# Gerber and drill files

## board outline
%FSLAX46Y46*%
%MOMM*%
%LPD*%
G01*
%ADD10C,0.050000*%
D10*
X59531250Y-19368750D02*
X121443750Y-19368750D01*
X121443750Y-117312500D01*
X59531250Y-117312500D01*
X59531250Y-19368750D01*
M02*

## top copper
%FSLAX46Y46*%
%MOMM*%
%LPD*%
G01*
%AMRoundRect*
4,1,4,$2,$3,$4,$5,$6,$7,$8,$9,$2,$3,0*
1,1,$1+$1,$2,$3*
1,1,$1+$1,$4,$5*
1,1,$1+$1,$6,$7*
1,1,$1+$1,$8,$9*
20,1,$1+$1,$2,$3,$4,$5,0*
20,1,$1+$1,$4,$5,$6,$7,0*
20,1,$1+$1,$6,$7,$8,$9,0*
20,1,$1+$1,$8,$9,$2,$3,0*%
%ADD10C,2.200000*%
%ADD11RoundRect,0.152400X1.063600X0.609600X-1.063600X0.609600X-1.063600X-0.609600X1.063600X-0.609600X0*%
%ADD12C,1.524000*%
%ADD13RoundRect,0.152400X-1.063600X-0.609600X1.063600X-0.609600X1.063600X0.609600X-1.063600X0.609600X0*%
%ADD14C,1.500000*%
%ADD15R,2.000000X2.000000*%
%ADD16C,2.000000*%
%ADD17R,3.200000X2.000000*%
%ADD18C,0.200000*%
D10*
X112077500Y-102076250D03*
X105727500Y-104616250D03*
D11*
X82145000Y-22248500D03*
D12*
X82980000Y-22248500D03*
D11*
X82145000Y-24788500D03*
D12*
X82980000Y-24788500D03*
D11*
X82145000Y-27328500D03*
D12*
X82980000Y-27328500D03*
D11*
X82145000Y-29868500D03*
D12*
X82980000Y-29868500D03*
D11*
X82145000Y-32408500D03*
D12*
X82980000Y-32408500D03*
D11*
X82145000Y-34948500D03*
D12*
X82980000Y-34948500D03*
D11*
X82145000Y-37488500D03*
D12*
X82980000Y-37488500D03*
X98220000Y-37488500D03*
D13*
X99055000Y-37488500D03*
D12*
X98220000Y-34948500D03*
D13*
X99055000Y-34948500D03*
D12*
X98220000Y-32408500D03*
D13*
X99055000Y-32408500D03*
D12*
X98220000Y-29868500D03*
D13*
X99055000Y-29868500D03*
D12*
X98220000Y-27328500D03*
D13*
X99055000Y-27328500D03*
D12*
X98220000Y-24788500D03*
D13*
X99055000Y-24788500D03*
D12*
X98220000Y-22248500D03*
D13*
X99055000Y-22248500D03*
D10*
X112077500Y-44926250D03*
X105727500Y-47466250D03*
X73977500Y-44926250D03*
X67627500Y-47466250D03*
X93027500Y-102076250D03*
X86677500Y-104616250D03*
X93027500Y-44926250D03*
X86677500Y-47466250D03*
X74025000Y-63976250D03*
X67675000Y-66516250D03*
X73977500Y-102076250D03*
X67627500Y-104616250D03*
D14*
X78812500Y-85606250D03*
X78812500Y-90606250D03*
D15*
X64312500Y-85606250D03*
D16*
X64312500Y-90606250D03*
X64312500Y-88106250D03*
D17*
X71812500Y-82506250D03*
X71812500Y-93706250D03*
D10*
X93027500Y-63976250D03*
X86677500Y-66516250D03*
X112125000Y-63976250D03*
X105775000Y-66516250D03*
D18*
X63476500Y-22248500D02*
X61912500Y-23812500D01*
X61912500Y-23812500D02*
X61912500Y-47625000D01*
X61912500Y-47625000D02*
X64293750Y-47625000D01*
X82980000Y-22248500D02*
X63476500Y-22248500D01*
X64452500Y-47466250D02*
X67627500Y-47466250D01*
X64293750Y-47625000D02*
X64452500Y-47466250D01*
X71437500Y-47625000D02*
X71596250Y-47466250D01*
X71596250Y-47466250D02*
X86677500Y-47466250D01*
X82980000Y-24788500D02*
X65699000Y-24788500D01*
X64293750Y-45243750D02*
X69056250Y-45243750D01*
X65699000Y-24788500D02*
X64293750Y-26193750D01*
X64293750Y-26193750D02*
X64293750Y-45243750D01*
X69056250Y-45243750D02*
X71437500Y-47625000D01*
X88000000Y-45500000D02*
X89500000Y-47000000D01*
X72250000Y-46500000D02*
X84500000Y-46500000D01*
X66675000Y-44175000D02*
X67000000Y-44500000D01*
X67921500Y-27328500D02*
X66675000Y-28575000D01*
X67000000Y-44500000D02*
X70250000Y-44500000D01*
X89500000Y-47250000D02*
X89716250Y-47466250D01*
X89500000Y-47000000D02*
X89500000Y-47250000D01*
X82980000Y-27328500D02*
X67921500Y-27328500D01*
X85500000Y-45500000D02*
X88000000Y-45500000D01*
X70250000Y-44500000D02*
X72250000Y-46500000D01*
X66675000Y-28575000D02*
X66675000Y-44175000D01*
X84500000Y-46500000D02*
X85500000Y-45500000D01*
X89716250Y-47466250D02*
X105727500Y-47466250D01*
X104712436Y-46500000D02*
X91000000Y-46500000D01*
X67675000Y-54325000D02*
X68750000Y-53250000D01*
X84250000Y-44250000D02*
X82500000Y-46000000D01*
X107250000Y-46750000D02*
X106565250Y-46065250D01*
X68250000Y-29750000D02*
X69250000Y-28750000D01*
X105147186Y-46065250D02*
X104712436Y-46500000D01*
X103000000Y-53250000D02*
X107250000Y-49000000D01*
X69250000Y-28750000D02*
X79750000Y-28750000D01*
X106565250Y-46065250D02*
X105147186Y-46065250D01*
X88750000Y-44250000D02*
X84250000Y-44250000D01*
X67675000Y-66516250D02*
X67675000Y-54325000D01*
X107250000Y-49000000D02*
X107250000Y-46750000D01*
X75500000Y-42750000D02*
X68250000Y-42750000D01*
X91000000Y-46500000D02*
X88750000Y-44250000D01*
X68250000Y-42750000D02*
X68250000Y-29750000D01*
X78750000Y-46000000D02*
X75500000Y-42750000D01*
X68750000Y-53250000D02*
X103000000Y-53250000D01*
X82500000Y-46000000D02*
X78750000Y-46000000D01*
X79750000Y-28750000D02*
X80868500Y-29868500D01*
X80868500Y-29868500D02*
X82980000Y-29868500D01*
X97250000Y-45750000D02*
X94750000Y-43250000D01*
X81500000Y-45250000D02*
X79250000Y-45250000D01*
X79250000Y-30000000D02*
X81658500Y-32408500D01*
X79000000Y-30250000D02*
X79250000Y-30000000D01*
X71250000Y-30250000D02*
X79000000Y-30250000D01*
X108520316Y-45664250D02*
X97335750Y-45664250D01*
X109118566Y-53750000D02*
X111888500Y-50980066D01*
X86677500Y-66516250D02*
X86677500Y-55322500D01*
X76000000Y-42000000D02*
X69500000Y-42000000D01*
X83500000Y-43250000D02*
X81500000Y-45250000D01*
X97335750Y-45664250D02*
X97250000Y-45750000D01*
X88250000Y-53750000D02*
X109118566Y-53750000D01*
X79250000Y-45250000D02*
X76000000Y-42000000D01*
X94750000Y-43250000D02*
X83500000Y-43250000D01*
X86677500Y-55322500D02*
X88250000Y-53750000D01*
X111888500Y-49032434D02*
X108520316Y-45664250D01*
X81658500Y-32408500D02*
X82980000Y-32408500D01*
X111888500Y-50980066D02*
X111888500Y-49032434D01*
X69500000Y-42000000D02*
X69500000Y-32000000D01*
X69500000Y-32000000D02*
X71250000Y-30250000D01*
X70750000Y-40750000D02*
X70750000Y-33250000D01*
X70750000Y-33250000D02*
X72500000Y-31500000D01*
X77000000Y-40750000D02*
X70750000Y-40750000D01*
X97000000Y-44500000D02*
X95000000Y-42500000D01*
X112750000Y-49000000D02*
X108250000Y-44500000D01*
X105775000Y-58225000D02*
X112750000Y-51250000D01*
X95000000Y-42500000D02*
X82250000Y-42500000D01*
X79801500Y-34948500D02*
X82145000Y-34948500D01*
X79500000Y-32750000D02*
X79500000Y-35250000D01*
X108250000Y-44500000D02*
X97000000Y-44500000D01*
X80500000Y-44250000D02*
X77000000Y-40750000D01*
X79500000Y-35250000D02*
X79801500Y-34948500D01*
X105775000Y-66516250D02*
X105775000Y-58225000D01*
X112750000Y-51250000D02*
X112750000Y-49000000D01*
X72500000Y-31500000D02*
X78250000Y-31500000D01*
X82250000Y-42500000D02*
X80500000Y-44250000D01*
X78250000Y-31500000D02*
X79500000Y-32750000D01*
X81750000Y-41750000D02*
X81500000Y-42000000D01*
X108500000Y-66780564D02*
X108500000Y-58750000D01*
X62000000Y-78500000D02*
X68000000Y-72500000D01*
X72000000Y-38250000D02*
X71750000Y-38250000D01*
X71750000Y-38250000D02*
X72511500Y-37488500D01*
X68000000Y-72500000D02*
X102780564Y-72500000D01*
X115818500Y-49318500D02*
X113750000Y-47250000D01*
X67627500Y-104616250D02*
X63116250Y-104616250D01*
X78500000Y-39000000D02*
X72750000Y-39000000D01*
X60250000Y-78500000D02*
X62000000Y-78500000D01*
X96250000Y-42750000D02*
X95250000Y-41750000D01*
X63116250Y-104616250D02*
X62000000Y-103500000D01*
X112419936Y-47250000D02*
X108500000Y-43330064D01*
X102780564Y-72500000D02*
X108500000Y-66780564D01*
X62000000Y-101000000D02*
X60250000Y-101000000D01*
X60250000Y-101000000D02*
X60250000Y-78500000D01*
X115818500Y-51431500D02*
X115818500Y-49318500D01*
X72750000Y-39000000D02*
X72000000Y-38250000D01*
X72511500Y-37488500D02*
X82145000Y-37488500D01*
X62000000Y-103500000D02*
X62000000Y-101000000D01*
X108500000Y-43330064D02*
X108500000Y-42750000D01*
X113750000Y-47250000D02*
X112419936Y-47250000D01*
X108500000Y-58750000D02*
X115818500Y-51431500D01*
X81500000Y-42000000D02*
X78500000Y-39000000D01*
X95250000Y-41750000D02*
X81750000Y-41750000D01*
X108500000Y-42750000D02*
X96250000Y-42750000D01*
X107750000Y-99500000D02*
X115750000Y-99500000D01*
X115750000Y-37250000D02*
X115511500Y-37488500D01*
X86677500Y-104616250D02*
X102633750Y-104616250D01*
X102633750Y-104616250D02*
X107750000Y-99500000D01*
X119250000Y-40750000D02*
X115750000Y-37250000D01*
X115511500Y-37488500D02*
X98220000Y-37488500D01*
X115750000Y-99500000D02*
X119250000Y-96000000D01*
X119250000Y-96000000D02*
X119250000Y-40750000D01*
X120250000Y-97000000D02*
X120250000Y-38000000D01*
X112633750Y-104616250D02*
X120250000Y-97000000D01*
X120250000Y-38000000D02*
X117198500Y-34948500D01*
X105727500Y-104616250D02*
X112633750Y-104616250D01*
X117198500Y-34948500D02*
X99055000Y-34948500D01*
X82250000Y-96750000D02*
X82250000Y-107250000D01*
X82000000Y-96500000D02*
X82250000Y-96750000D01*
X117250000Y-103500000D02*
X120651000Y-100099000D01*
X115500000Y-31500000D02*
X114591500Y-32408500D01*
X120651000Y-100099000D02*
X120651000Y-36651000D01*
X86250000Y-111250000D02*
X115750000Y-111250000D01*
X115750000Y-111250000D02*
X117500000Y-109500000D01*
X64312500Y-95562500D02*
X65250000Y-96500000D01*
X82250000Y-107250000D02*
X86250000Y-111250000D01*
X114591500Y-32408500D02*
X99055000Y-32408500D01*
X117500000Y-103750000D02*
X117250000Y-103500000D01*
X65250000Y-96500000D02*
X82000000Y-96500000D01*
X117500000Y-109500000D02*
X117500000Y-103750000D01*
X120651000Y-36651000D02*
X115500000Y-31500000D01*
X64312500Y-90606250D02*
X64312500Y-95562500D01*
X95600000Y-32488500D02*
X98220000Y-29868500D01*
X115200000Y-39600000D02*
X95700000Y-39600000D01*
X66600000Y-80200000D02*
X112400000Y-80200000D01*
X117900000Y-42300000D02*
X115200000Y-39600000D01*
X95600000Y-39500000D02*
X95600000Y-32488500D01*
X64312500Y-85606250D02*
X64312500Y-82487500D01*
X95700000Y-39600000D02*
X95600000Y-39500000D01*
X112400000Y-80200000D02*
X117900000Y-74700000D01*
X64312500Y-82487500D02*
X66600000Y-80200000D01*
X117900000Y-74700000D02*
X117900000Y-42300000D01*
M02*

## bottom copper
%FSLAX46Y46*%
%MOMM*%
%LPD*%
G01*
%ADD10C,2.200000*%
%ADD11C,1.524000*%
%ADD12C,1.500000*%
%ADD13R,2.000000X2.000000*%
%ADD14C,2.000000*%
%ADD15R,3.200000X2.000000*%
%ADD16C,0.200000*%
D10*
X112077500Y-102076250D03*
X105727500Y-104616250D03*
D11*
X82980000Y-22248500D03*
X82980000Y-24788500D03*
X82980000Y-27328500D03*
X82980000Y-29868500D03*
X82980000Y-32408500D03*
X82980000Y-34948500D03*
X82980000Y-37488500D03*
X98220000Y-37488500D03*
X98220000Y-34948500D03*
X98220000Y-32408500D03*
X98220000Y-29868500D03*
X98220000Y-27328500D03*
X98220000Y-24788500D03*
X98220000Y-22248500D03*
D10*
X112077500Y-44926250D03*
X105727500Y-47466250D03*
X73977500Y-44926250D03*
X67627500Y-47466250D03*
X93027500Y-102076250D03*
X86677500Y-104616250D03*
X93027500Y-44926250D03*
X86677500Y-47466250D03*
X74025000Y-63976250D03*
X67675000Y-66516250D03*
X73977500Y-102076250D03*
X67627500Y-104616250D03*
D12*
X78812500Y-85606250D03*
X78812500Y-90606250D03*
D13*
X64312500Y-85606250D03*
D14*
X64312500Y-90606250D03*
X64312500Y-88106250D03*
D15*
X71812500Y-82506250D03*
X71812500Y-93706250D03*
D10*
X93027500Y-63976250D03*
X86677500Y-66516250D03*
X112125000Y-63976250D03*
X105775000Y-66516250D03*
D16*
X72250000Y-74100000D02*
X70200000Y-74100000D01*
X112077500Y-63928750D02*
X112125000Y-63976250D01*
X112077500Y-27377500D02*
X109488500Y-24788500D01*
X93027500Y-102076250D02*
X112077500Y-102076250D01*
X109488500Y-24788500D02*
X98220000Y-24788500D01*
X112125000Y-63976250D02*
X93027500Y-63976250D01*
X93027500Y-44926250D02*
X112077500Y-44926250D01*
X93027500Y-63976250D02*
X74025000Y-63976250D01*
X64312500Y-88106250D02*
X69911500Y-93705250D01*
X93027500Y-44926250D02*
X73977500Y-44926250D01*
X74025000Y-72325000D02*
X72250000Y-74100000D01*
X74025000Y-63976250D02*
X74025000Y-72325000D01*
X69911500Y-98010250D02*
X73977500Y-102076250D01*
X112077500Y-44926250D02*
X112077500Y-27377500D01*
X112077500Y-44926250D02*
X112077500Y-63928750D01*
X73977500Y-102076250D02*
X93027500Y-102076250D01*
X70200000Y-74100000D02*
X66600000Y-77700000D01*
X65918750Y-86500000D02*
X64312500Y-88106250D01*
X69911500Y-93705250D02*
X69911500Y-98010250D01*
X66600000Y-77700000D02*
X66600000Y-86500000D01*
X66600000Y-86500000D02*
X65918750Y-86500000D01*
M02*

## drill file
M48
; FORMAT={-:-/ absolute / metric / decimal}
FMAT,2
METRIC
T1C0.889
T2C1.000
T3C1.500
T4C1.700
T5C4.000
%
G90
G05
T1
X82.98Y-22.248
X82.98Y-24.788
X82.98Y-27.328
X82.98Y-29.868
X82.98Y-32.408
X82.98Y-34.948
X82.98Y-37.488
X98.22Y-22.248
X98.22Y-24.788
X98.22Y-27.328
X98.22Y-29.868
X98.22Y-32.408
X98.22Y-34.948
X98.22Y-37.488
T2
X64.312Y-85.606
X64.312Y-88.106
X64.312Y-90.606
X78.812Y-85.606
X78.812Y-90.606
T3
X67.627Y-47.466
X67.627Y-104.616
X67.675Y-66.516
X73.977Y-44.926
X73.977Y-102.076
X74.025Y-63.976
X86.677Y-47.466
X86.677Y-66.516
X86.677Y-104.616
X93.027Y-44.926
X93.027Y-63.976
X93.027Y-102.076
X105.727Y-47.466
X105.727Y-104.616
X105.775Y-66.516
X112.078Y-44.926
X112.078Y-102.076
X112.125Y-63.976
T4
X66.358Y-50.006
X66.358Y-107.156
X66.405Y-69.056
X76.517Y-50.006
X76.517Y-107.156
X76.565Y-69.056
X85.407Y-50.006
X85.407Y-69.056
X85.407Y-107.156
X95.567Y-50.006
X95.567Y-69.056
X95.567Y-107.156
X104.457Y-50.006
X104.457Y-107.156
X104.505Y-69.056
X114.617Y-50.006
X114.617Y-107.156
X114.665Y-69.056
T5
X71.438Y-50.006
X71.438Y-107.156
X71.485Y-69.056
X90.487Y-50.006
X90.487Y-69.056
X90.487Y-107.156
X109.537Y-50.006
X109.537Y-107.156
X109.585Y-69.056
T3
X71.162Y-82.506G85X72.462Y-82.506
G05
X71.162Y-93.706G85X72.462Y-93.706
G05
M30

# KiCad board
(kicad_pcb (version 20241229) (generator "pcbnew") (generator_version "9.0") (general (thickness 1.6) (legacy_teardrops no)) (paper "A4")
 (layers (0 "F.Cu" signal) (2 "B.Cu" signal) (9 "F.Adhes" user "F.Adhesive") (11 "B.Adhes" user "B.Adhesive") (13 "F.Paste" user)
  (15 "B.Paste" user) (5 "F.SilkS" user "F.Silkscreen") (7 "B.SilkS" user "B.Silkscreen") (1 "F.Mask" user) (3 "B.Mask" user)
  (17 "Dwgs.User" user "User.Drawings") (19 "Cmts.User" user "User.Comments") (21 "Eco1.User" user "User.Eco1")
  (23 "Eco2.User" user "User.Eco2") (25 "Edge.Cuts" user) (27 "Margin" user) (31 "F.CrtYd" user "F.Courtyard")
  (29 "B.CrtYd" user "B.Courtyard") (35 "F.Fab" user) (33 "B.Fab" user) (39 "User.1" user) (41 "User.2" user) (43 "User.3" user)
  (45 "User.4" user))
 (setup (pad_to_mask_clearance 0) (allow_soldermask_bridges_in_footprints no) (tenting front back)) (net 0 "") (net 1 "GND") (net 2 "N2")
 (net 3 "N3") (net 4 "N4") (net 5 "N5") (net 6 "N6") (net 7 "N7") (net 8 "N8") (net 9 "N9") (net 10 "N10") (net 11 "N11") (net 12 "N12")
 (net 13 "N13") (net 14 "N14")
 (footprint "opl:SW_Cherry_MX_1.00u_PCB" (layer "F.Cu") (at 112.0775 102.07625)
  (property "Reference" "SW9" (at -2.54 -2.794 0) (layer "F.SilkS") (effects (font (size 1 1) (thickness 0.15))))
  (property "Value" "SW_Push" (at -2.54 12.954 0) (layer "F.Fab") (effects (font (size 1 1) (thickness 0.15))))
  (pad "" np_thru_hole circle (at -7.62 5.08) (size 1.7 1.7) (drill 1.7) (layers "*.Cu" "*.Mask"))
  (pad "" np_thru_hole circle (at -2.54 5.08) (size 4 4) (drill 4) (layers "*.Cu" "*.Mask"))
  (pad "" np_thru_hole circle (at 2.54 5.08) (size 1.7 1.7) (drill 1.7) (layers "*.Cu" "*.Mask"))
  (pad "1" thru_hole circle (at 0 0) (size 2.2 2.2) (drill 1.5) (layers "*.Cu" "*.Mask") (remove_unused_layers no) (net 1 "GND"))
  (pad "2" thru_hole circle (at -6.35 2.54) (size 2.2 2.2) (drill 1.5) (layers "*.Cu" "*.Mask") (remove_unused_layers no) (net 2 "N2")))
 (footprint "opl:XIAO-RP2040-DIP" (layer "F.Cu") (at 90.6 29.8685)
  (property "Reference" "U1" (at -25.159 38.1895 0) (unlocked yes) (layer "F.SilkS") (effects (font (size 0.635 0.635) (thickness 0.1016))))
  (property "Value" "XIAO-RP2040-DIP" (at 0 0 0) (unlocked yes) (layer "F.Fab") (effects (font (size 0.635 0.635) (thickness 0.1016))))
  (pad "1" smd roundrect (at -8.455 -7.62 180) (size 2.432 1.524) (layers "F.Cu" "F.Mask") (roundrect_rratio 0.1) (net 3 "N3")
   (thermal_bridge_angle 45))
  (pad "1" thru_hole circle (at -7.62 -7.62 180) (size 1.524 1.524) (drill 0.889) (layers "*.Cu" "*.Mask") (remove_unused_layers no)
   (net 3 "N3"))
  (pad "2" smd roundrect (at -8.455 -5.08 180) (size 2.432 1.524) (layers "F.Cu" "F.Mask") (roundrect_rratio 0.1) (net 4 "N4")
   (thermal_bridge_angle 45))
  (pad "2" thru_hole circle (at -7.62 -5.08 180) (size 1.524 1.524) (drill 0.889) (layers "*.Cu" "*.Mask") (remove_unused_layers no)
   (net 4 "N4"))
  (pad "3" smd roundrect (at -8.455 -2.54 180) (size 2.432 1.524) (layers "F.Cu" "F.Mask") (roundrect_rratio 0.1) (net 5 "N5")
   (thermal_bridge_angle 45))
  (pad "3" thru_hole circle (at -7.62 -2.54 180) (size 1.524 1.524) (drill 0.889) (layers "*.Cu" "*.Mask") (remove_unused_layers no)
   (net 5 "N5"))
  (pad "4" smd roundrect (at -8.455 0 180) (size 2.432 1.524) (layers "F.Cu" "F.Mask") (roundrect_rratio 0.1) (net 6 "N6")
   (thermal_bridge_angle 45))
  (pad "4" thru_hole circle (at -7.62 0 180) (size 1.524 1.524) (drill 0.889) (layers "*.Cu" "*.Mask") (remove_unused_layers no)
   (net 6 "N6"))
  (pad "5" smd roundrect (at -8.455 2.54 180) (size 2.432 1.524) (layers "F.Cu" "F.Mask") (roundrect_rratio 0.1) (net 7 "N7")
   (thermal_bridge_angle 45))
  (pad "5" thru_hole circle (at -7.62 2.54 180) (size 1.524 1.524) (drill 0.889) (layers "*.Cu" "*.Mask") (remove_unused_layers no)
   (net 7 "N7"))
  (pad "6" smd roundrect (at -8.455 5.08 180) (size 2.432 1.524) (layers "F.Cu" "F.Mask") (roundrect_rratio 0.1) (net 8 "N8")
   (thermal_bridge_angle 45))
  (pad "6" thru_hole circle (at -7.62 5.08 180) (size 1.524 1.524) (drill 0.889) (layers "*.Cu" "*.Mask") (remove_unused_layers no)
   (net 8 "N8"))
  (pad "7" smd roundrect (at -8.455 7.62 180) (size 2.432 1.524) (layers "F.Cu" "F.Mask") (roundrect_rratio 0.1) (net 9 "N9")
   (thermal_bridge_angle 45))
  (pad "7" thru_hole circle (at -7.62 7.62 180) (size 1.524 1.524) (drill 0.889) (layers "*.Cu" "*.Mask") (remove_unused_layers no)
   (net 9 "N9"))
  (pad "8" thru_hole circle (at 7.62 7.62) (size 1.524 1.524) (drill 0.889) (layers "*.Cu" "*.Mask") (remove_unused_layers no)
   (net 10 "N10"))
  (pad "8" smd roundrect (at 8.455 7.62) (size 2.432 1.524) (layers "F.Cu" "F.Mask") (roundrect_rratio 0.1) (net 10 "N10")
   (thermal_bridge_angle 45))
  (pad "9" thru_hole circle (at 7.62 5.08) (size 1.524 1.524) (drill 0.889) (layers "*.Cu" "*.Mask") (remove_unused_layers no) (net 2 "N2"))
  (pad "9" smd roundrect (at 8.455 5.08) (size 2.432 1.524) (layers "F.Cu" "F.Mask") (roundrect_rratio 0.1) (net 2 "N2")
   (thermal_bridge_angle 45))
  (pad "10" thru_hole circle (at 7.62 2.54) (size 1.524 1.524) (drill 0.889) (layers "*.Cu" "*.Mask") (remove_unused_layers no)
   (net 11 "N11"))
  (pad "10" smd roundrect (at 8.455 2.54) (size 2.432 1.524) (layers "F.Cu" "F.Mask") (roundrect_rratio 0.1) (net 11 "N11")
   (thermal_bridge_angle 45))
  (pad "11" thru_hole circle (at 7.62 0) (size 1.524 1.524) (drill 0.889) (layers "*.Cu" "*.Mask") (remove_unused_layers no) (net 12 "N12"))
  (pad "11" smd roundrect (at 8.455 0) (size 2.432 1.524) (layers "F.Cu" "F.Mask") (roundrect_rratio 0.1) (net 12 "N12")
   (thermal_bridge_angle 45))
  (pad "12" thru_hole circle (at 7.62 -2.54) (size 1.524 1.524) (drill 0.889) (layers "*.Cu" "*.Mask") (remove_unused_layers no)
   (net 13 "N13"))
  (pad "12" smd roundrect (at 8.455 -2.54) (size 2.432 1.524) (layers "F.Cu" "F.Mask") (roundrect_rratio 0.1) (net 13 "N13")
   (thermal_bridge_angle 45))
  (pad "13" thru_hole circle (at 7.62 -5.08) (size 1.524 1.524) (drill 0.889) (layers "*.Cu" "*.Mask") (remove_unused_layers no)
   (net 1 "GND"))
  (pad "13" smd roundrect (at 8.455 -5.08) (size 2.432 1.524) (layers "F.Cu" "F.Mask") (roundrect_rratio 0.1) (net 1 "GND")
   (thermal_bridge_angle 45))
  (pad "14" thru_hole circle (at 7.62 -7.62) (size 1.524 1.524) (drill 0.889) (layers "*.Cu" "*.Mask") (remove_unused_layers no)
   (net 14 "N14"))
  (pad "14" smd roundrect (at 8.455 -7.62) (size 2.432 1.524) (layers "F.Cu" "F.Mask") (roundrect_rratio 0.1) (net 14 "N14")
   (thermal_bridge_angle 45)))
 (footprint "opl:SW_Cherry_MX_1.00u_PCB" (layer "F.Cu") (at 112.0775 44.92625)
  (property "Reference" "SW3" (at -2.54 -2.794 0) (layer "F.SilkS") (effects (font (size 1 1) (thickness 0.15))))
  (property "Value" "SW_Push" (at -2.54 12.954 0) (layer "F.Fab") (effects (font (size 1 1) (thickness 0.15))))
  (pad "" np_thru_hole circle (at -7.62 5.08) (size 1.7 1.7) (drill 1.7) (layers "*.Cu" "*.Mask"))
  (pad "" np_thru_hole circle (at -2.54 5.08) (size 4 4) (drill 4) (layers "*.Cu" "*.Mask"))
  (pad "" np_thru_hole circle (at 2.54 5.08) (size 1.7 1.7) (drill 1.7) (layers "*.Cu" "*.Mask"))
  (pad "1" thru_hole circle (at 0 0) (size 2.2 2.2) (drill 1.5) (layers "*.Cu" "*.Mask") (remove_unused_layers no) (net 1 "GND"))
  (pad "2" thru_hole circle (at -6.35 2.54) (size 2.2 2.2) (drill 1.5) (layers "*.Cu" "*.Mask") (remove_unused_layers no) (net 5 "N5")))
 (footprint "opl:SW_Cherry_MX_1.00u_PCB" (layer "F.Cu") (at 73.9775 44.92625)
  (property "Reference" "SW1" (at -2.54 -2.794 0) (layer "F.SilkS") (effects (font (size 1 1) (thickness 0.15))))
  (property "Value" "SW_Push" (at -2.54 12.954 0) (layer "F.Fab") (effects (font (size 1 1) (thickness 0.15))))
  (pad "" np_thru_hole circle (at -7.62 5.08) (size 1.7 1.7) (drill 1.7) (layers "*.Cu" "*.Mask"))
  (pad "" np_thru_hole circle (at -2.54 5.08) (size 4 4) (drill 4) (layers "*.Cu" "*.Mask"))
  (pad "" np_thru_hole circle (at 2.54 5.08) (size 1.7 1.7) (drill 1.7) (layers "*.Cu" "*.Mask"))
  (pad "1" thru_hole circle (at 0 0) (size 2.2 2.2) (drill 1.5) (layers "*.Cu" "*.Mask") (remove_unused_layers no) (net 1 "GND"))
  (pad "2" thru_hole circle (at -6.35 2.54) (size 2.2 2.2) (drill 1.5) (layers "*.Cu" "*.Mask") (remove_unused_layers no) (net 3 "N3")))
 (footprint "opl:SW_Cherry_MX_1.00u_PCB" (layer "F.Cu") (at 93.0275 102.07625)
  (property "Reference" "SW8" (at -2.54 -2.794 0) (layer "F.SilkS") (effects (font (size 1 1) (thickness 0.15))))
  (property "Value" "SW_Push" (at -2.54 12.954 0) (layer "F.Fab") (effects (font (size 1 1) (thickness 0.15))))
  (pad "" np_thru_hole circle (at -7.62 5.08) (size 1.7 1.7) (drill 1.7) (layers "*.Cu" "*.Mask"))
  (pad "" np_thru_hole circle (at -2.54 5.08) (size 4 4) (drill 4) (layers "*.Cu" "*.Mask"))
  (pad "" np_thru_hole circle (at 2.54 5.08) (size 1.7 1.7) (drill 1.7) (layers "*.Cu" "*.Mask"))
  (pad "1" thru_hole circle (at 0 0) (size 2.2 2.2) (drill 1.5) (layers "*.Cu" "*.Mask") (remove_unused_layers no) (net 1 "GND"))
  (pad "2" thru_hole circle (at -6.35 2.54) (size 2.2 2.2) (drill 1.5) (layers "*.Cu" "*.Mask") (remove_unused_layers no) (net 10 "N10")))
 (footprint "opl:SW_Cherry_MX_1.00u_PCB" (layer "F.Cu") (at 93.0275 44.92625)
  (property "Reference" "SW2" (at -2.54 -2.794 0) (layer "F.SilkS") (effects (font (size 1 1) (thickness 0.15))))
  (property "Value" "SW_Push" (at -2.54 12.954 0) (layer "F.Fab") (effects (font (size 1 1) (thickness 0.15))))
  (pad "" np_thru_hole circle (at -7.62 5.08) (size 1.7 1.7) (drill 1.7) (layers "*.Cu" "*.Mask"))
  (pad "" np_thru_hole circle (at -2.54 5.08) (size 4 4) (drill 4) (layers "*.Cu" "*.Mask"))
  (pad "" np_thru_hole circle (at 2.54 5.08) (size 1.7 1.7) (drill 1.7) (layers "*.Cu" "*.Mask"))
  (pad "1" thru_hole circle (at 0 0) (size 2.2 2.2) (drill 1.5) (layers "*.Cu" "*.Mask") (remove_unused_layers no) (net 1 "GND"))
  (pad "2" thru_hole circle (at -6.35 2.54) (size 2.2 2.2) (drill 1.5) (layers "*.Cu" "*.Mask") (remove_unused_layers no) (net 4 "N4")))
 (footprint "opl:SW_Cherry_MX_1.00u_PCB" (layer "F.Cu") (at 74.025 63.97625)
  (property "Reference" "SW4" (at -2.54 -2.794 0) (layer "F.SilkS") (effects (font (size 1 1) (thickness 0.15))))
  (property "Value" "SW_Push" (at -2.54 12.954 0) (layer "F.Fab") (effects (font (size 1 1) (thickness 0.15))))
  (pad "" np_thru_hole circle (at -7.62 5.08) (size 1.7 1.7) (drill 1.7) (layers "*.Cu" "*.Mask"))
  (pad "" np_thru_hole circle (at -2.54 5.08) (size 4 4) (drill 4) (layers "*.Cu" "*.Mask"))
  (pad "" np_thru_hole circle (at 2.54 5.08) (size 1.7 1.7) (drill 1.7) (layers "*.Cu" "*.Mask"))
  (pad "1" thru_hole circle (at 0 0) (size 2.2 2.2) (drill 1.5) (layers "*.Cu" "*.Mask") (remove_unused_layers no) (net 1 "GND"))
  (pad "2" thru_hole circle (at -6.35 2.54) (size 2.2 2.2) (drill 1.5) (layers "*.Cu" "*.Mask") (remove_unused_layers no) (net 6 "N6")))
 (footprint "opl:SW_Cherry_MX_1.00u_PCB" (layer "F.Cu") (at 73.9775 102.07625)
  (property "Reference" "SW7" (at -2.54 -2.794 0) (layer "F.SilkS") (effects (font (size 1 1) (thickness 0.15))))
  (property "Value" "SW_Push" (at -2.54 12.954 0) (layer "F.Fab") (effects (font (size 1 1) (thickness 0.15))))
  (pad "" np_thru_hole circle (at -7.62 5.08) (size 1.7 1.7) (drill 1.7) (layers "*.Cu" "*.Mask"))
  (pad "" np_thru_hole circle (at -2.54 5.08) (size 4 4) (drill 4) (layers "*.Cu" "*.Mask"))
  (pad "" np_thru_hole circle (at 2.54 5.08) (size 1.7 1.7) (drill 1.7) (layers "*.Cu" "*.Mask"))
  (pad "1" thru_hole circle (at 0 0) (size 2.2 2.2) (drill 1.5) (layers "*.Cu" "*.Mask") (remove_unused_layers no) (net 1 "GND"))
  (pad "2" thru_hole circle (at -6.35 2.54) (size 2.2 2.2) (drill 1.5) (layers "*.Cu" "*.Mask") (remove_unused_layers no) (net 9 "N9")))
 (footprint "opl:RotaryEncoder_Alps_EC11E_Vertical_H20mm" (layer "F.Cu") (at 64.3125 85.60625)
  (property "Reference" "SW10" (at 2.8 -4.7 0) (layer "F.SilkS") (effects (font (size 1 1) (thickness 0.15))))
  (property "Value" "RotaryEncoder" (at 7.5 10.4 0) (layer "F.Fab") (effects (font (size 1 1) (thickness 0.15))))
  (pad "" thru_hole circle (at 14.5 0) (size 1.5 1.5) (drill 1) (layers "*.Cu" "*.Mask") (remove_unused_layers no))
  (pad "" thru_hole circle (at 14.5 5) (size 1.5 1.5) (drill 1) (layers "*.Cu" "*.Mask") (remove_unused_layers no))
  (pad "A" thru_hole rect (at 0 0) (size 2 2) (drill 1) (layers "*.Cu" "*.Mask") (remove_unused_layers no) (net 12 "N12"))
  (pad "B" thru_hole circle (at 0 5) (size 2 2) (drill 1) (layers "*.Cu" "*.Mask") (remove_unused_layers no) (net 11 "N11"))
  (pad "C" thru_hole circle (at 0 2.5) (size 2 2) (drill 1) (layers "*.Cu" "*.Mask") (remove_unused_layers no) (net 1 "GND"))
  (pad "MP" thru_hole rect (at 7.5 -3.1) (size 3.2 2) (drill oval 2.8 1.5) (layers "*.Cu" "*.Mask") (remove_unused_layers no))
  (pad "MP" thru_hole rect (at 7.5 8.1) (size 3.2 2) (drill oval 2.8 1.5) (layers "*.Cu" "*.Mask") (remove_unused_layers no)))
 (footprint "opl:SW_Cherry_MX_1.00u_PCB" (layer "F.Cu") (at 93.0275 63.97625)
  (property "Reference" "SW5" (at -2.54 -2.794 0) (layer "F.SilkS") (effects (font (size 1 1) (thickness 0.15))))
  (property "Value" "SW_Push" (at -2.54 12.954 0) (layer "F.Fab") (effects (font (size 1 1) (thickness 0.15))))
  (pad "" np_thru_hole circle (at -7.62 5.08) (size 1.7 1.7) (drill 1.7) (layers "*.Cu" "*.Mask"))
  (pad "" np_thru_hole circle (at -2.54 5.08) (size 4 4) (drill 4) (layers "*.Cu" "*.Mask"))
  (pad "" np_thru_hole circle (at 2.54 5.08) (size 1.7 1.7) (drill 1.7) (layers "*.Cu" "*.Mask"))
  (pad "1" thru_hole circle (at 0 0) (size 2.2 2.2) (drill 1.5) (layers "*.Cu" "*.Mask") (remove_unused_layers no) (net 1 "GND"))
  (pad "2" thru_hole circle (at -6.35 2.54) (size 2.2 2.2) (drill 1.5) (layers "*.Cu" "*.Mask") (remove_unused_layers no) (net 7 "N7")))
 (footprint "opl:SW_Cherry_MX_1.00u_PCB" (layer "F.Cu") (at 112.125 63.97625)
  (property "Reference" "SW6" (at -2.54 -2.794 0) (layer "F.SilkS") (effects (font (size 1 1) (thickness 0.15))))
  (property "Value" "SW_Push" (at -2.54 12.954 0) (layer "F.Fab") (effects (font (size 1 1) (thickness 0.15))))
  (pad "" np_thru_hole circle (at -7.62 5.08) (size 1.7 1.7) (drill 1.7) (layers "*.Cu" "*.Mask"))
  (pad "" np_thru_hole circle (at -2.54 5.08) (size 4 4) (drill 4) (layers "*.Cu" "*.Mask"))
  (pad "" np_thru_hole circle (at 2.54 5.08) (size 1.7 1.7) (drill 1.7) (layers "*.Cu" "*.Mask"))
  (pad "1" thru_hole circle (at 0 0) (size 2.2 2.2) (drill 1.5) (layers "*.Cu" "*.Mask") (remove_unused_layers no) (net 1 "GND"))
  (pad "2" thru_hole circle (at -6.35 2.54) (size 2.2 2.2) (drill 1.5) (layers "*.Cu" "*.Mask") (remove_unused_layers no) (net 8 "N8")))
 (gr_rect (start 59.53125 19.36875) (end 121.44375 117.3125) (stroke (width 0.05) (type default)) (fill no) (layer "Edge.Cuts"))
 (segment (start 72.25 74.1) (end 70.2 74.1) (width 0.2) (layer "B.Cu") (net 1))
 (segment (start 112.0775 63.92875) (end 112.125 63.97625) (width 0.2) (layer "B.Cu") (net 1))
 (segment (start 112.0775 27.3775) (end 109.4885 24.7885) (width 0.2) (layer "B.Cu") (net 1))
 (segment (start 93.0275 102.07625) (end 112.0775 102.07625) (width 0.2) (layer "B.Cu") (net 1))
 (segment (start 109.4885 24.7885) (end 98.22 24.7885) (width 0.2) (layer "B.Cu") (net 1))
 (segment (start 112.125 63.97625) (end 93.0275 63.97625) (width 0.2) (layer "B.Cu") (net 1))
 (segment (start 93.0275 44.92625) (end 112.0775 44.92625) (width 0.2) (layer "B.Cu") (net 1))
 (segment (start 93.0275 63.97625) (end 74.025 63.97625) (width 0.2) (layer "B.Cu") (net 1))
 (segment (start 64.3125 88.10625) (end 69.9115 93.70525) (width 0.2) (layer "B.Cu") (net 1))
 (segment (start 93.0275 44.92625) (end 73.9775 44.92625) (width 0.2) (layer "B.Cu") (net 1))
 (segment (start 74.025 72.325) (end 72.25 74.1) (width 0.2) (layer "B.Cu") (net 1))
 (segment (start 74.025 63.97625) (end 74.025 72.325) (width 0.2) (layer "B.Cu") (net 1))
 (segment (start 69.9115 98.01025) (end 73.9775 102.07625) (width 0.2) (layer "B.Cu") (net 1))
 (segment (start 112.0775 44.92625) (end 112.0775 27.3775) (width 0.2) (layer "B.Cu") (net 1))
 (segment (start 112.0775 44.92625) (end 112.0775 63.92875) (width 0.2) (layer "B.Cu") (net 1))
 (segment (start 73.9775 102.07625) (end 93.0275 102.07625) (width 0.2) (layer "B.Cu") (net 1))
 (segment (start 70.2 74.1) (end 66.6 77.7) (width 0.2) (layer "B.Cu") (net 1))
 (segment (start 65.91875 86.5) (end 64.3125 88.10625) (width 0.2) (layer "B.Cu") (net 1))
 (segment (start 69.9115 93.70525) (end 69.9115 98.01025) (width 0.2) (layer "B.Cu") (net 1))
 (segment (start 66.6 77.7) (end 66.6 86.5) (width 0.2) (layer "B.Cu") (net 1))
 (segment (start 66.6 86.5) (end 65.91875 86.5) (width 0.2) (layer "B.Cu") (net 1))
 (segment (start 63.4765 22.2485) (end 61.9125 23.8125) (width 0.2) (layer "F.Cu") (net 3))
 (segment (start 61.9125 23.8125) (end 61.9125 47.625) (width 0.2) (layer "F.Cu") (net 3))
 (segment (start 61.9125 47.625) (end 64.29375 47.625) (width 0.2) (layer "F.Cu") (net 3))
 (segment (start 82.98 22.2485) (end 63.4765 22.2485) (width 0.2) (layer "F.Cu") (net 3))
 (segment (start 64.4525 47.46625) (end 67.6275 47.46625) (width 0.2) (layer "F.Cu") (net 3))
 (segment (start 64.29375 47.625) (end 64.4525 47.46625) (width 0.2) (layer "F.Cu") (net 3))
 (segment (start 71.4375 47.625) (end 71.59625 47.46625) (width 0.2) (layer "F.Cu") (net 4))
 (segment (start 71.59625 47.46625) (end 86.6775 47.46625) (width 0.2) (layer "F.Cu") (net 4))
 (segment (start 82.98 24.7885) (end 65.699 24.7885) (width 0.2) (layer "F.Cu") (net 4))
 (segment (start 64.29375 45.24375) (end 69.05625 45.24375) (width 0.2) (layer "F.Cu") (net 4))
 (segment (start 65.699 24.7885) (end 64.29375 26.19375) (width 0.2) (layer "F.Cu") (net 4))
 (segment (start 64.29375 26.19375) (end 64.29375 45.24375) (width 0.2) (layer "F.Cu") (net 4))
 (segment (start 69.05625 45.24375) (end 71.4375 47.625) (width 0.2) (layer "F.Cu") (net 4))
 (segment (start 88 45.5) (end 89.5 47) (width 0.2) (layer "F.Cu") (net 5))
 (segment (start 72.25 46.5) (end 84.5 46.5) (width 0.2) (layer "F.Cu") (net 5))
 (segment (start 66.675 44.175) (end 67 44.5) (width 0.2) (layer "F.Cu") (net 5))
 (segment (start 67.9215 27.3285) (end 66.675 28.575) (width 0.2) (layer "F.Cu") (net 5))
 (segment (start 67 44.5) (end 70.25 44.5) (width 0.2) (layer "F.Cu") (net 5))
 (segment (start 89.5 47.25) (end 89.71625 47.46625) (width 0.2) (layer "F.Cu") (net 5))
 (segment (start 89.5 47) (end 89.5 47.25) (width 0.2) (layer "F.Cu") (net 5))
 (segment (start 82.98 27.3285) (end 67.9215 27.3285) (width 0.2) (layer "F.Cu") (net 5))
 (segment (start 85.5 45.5) (end 88 45.5) (width 0.2) (layer "F.Cu") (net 5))
 (segment (start 70.25 44.5) (end 72.25 46.5) (width 0.2) (layer "F.Cu") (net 5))
 (segment (start 66.675 28.575) (end 66.675 44.175) (width 0.2) (layer "F.Cu") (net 5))
 (segment (start 84.5 46.5) (end 85.5 45.5) (width 0.2) (layer "F.Cu") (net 5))
 (segment (start 89.71625 47.46625) (end 105.7275 47.46625) (width 0.2) (layer "F.Cu") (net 5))
 (segment (start 104.712436 46.5) (end 91 46.5) (width 0.2) (layer "F.Cu") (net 6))
 (segment (start 67.675 54.325) (end 68.75 53.25) (width 0.2) (layer "F.Cu") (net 6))
 (segment (start 84.25 44.25) (end 82.5 46) (width 0.2) (layer "F.Cu") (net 6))
 (segment (start 107.25 46.75) (end 106.56525 46.06525) (width 0.2) (layer "F.Cu") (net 6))
 (segment (start 68.25 29.75) (end 69.25 28.75) (width 0.2) (layer "F.Cu") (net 6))
 (segment (start 105.147186 46.06525) (end 104.712436 46.5) (width 0.2) (layer "F.Cu") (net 6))
 (segment (start 103 53.25) (end 107.25 49) (width 0.2) (layer "F.Cu") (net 6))
 (segment (start 69.25 28.75) (end 79.75 28.75) (width 0.2) (layer "F.Cu") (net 6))
 (segment (start 106.56525 46.06525) (end 105.147186 46.06525) (width 0.2) (layer "F.Cu") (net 6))
 (segment (start 88.75 44.25) (end 84.25 44.25) (width 0.2) (layer "F.Cu") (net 6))
 (segment (start 67.675 66.51625) (end 67.675 54.325) (width 0.2) (layer "F.Cu") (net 6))
 (segment (start 107.25 49) (end 107.25 46.75) (width 0.2) (layer "F.Cu") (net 6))
 (segment (start 75.5 42.75) (end 68.25 42.75) (width 0.2) (layer "F.Cu") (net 6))
 (segment (start 91 46.5) (end 88.75 44.25) (width 0.2) (layer "F.Cu") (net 6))
 (segment (start 68.25 42.75) (end 68.25 29.75) (width 0.2) (layer "F.Cu") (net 6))
 (segment (start 78.75 46) (end 75.5 42.75) (width 0.2) (layer "F.Cu") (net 6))
 (segment (start 68.75 53.25) (end 103 53.25) (width 0.2) (layer "F.Cu") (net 6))
 (segment (start 82.5 46) (end 78.75 46) (width 0.2) (layer "F.Cu") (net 6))
 (segment (start 79.75 28.75) (end 80.8685 29.8685) (width 0.2) (layer "F.Cu") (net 6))
 (segment (start 80.8685 29.8685) (end 82.98 29.8685) (width 0.2) (layer "F.Cu") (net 6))
 (segment (start 97.25 45.75) (end 94.75 43.25) (width 0.2) (layer "F.Cu") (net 7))
 (segment (start 81.5 45.25) (end 79.25 45.25) (width 0.2) (layer "F.Cu") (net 7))
 (segment (start 79.25 30) (end 81.6585 32.4085) (width 0.2) (layer "F.Cu") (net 7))
 (segment (start 79 30.25) (end 79.25 30) (width 0.2) (layer "F.Cu") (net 7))
 (segment (start 71.25 30.25) (end 79 30.25) (width 0.2) (layer "F.Cu") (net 7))
 (segment (start 108.520316 45.66425) (end 97.33575 45.66425) (width 0.2) (layer "F.Cu") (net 7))
 (segment (start 109.118566 53.75) (end 111.8885 50.980066) (width 0.2) (layer "F.Cu") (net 7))
 (segment (start 86.6775 66.51625) (end 86.6775 55.3225) (width 0.2) (layer "F.Cu") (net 7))
 (segment (start 76 42) (end 69.5 42) (width 0.2) (layer "F.Cu") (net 7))
 (segment (start 83.5 43.25) (end 81.5 45.25) (width 0.2) (layer "F.Cu") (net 7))
 (segment (start 97.33575 45.66425) (end 97.25 45.75) (width 0.2) (layer "F.Cu") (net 7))
 (segment (start 88.25 53.75) (end 109.118566 53.75) (width 0.2) (layer "F.Cu") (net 7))
 (segment (start 79.25 45.25) (end 76 42) (width 0.2) (layer "F.Cu") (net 7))
 (segment (start 94.75 43.25) (end 83.5 43.25) (width 0.2) (layer "F.Cu") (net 7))
 (segment (start 86.6775 55.3225) (end 88.25 53.75) (width 0.2) (layer "F.Cu") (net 7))
 (segment (start 111.8885 49.032434) (end 108.520316 45.66425) (width 0.2) (layer "F.Cu") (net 7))
 (segment (start 81.6585 32.4085) (end 82.98 32.4085) (width 0.2) (layer "F.Cu") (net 7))
 (segment (start 111.8885 50.980066) (end 111.8885 49.032434) (width 0.2) (layer "F.Cu") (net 7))
 (segment (start 69.5 42) (end 69.5 32) (width 0.2) (layer "F.Cu") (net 7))
 (segment (start 69.5 32) (end 71.25 30.25) (width 0.2) (layer "F.Cu") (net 7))
 (segment (start 70.75 40.75) (end 70.75 33.25) (width 0.2) (layer "F.Cu") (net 8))
 (segment (start 70.75 33.25) (end 72.5 31.5) (width 0.2) (layer "F.Cu") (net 8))
 (segment (start 77 40.75) (end 70.75 40.75) (width 0.2) (layer "F.Cu") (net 8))
 (segment (start 97 44.5) (end 95 42.5) (width 0.2) (layer "F.Cu") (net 8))
 (segment (start 112.75 49) (end 108.25 44.5) (width 0.2) (layer "F.Cu") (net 8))
 (segment (start 105.775 58.225) (end 112.75 51.25) (width 0.2) (layer "F.Cu") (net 8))
 (segment (start 95 42.5) (end 82.25 42.5) (width 0.2) (layer "F.Cu") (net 8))
 (segment (start 79.8015 34.9485) (end 82.145 34.9485) (width 0.2) (layer "F.Cu") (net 8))
 (segment (start 79.5 32.75) (end 79.5 35.25) (width 0.2) (layer "F.Cu") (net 8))
 (segment (start 108.25 44.5) (end 97 44.5) (width 0.2) (layer "F.Cu") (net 8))
 (segment (start 80.5 44.25) (end 77 40.75) (width 0.2) (layer "F.Cu") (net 8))
 (segment (start 79.5 35.25) (end 79.8015 34.9485) (width 0.2) (layer "F.Cu") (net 8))
 (segment (start 105.775 66.51625) (end 105.775 58.225) (width 0.2) (layer "F.Cu") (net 8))
 (segment (start 112.75 51.25) (end 112.75 49) (width 0.2) (layer "F.Cu") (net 8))
 (segment (start 72.5 31.5) (end 78.25 31.5) (width 0.2) (layer "F.Cu") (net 8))
 (segment (start 82.25 42.5) (end 80.5 44.25) (width 0.2) (layer "F.Cu") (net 8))
 (segment (start 78.25 31.5) (end 79.5 32.75) (width 0.2) (layer "F.Cu") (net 8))
 (segment (start 81.75 41.75) (end 81.5 42) (width 0.2) (layer "F.Cu") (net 9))
 (segment (start 108.5 66.780564) (end 108.5 58.75) (width 0.2) (layer "F.Cu") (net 9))
 (segment (start 62 78.5) (end 68 72.5) (width 0.2) (layer "F.Cu") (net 9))
 (segment (start 72 38.25) (end 71.75 38.25) (width 0.2) (layer "F.Cu") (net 9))
 (segment (start 71.75 38.25) (end 72.5115 37.4885) (width 0.2) (layer "F.Cu") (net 9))
 (segment (start 68 72.5) (end 102.780564 72.5) (width 0.2) (layer "F.Cu") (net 9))
 (segment (start 115.8185 49.3185) (end 113.75 47.25) (width 0.2) (layer "F.Cu") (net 9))
 (segment (start 67.6275 104.61625) (end 63.11625 104.61625) (width 0.2) (layer "F.Cu") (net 9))
 (segment (start 78.5 39) (end 72.75 39) (width 0.2) (layer "F.Cu") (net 9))
 (segment (start 60.25 78.5) (end 62 78.5) (width 0.2) (layer "F.Cu") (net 9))
 (segment (start 96.25 42.75) (end 95.25 41.75) (width 0.2) (layer "F.Cu") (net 9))
 (segment (start 63.11625 104.61625) (end 62 103.5) (width 0.2) (layer "F.Cu") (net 9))
 (segment (start 112.419936 47.25) (end 108.5 43.330064) (width 0.2) (layer "F.Cu") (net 9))
 (segment (start 102.780564 72.5) (end 108.5 66.780564) (width 0.2) (layer "F.Cu") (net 9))
 (segment (start 62 101) (end 60.25 101) (width 0.2) (layer "F.Cu") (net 9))
 (segment (start 60.25 101) (end 60.25 78.5) (width 0.2) (layer "F.Cu") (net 9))
 (segment (start 115.8185 51.4315) (end 115.8185 49.3185) (width 0.2) (layer "F.Cu") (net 9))
 (segment (start 72.75 39) (end 72 38.25) (width 0.2) (layer "F.Cu") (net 9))
 (segment (start 72.5115 37.4885) (end 82.145 37.4885) (width 0.2) (layer "F.Cu") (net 9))
 (segment (start 62 103.5) (end 62 101) (width 0.2) (layer "F.Cu") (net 9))
 (segment (start 108.5 43.330064) (end 108.5 42.75) (width 0.2) (layer "F.Cu") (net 9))
 (segment (start 113.75 47.25) (end 112.419936 47.25) (width 0.2) (layer "F.Cu") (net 9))
 (segment (start 108.5 58.75) (end 115.8185 51.4315) (width 0.2) (layer "F.Cu") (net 9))
 (segment (start 81.5 42) (end 78.5 39) (width 0.2) (layer "F.Cu") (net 9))
 (segment (start 95.25 41.75) (end 81.75 41.75) (width 0.2) (layer "F.Cu") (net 9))
 (segment (start 108.5 42.75) (end 96.25 42.75) (width 0.2) (layer "F.Cu") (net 9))
 (segment (start 107.75 99.5) (end 115.75 99.5) (width 0.2) (layer "F.Cu") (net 10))
 (segment (start 115.75 37.25) (end 115.5115 37.4885) (width 0.2) (layer "F.Cu") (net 10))
 (segment (start 86.6775 104.61625) (end 102.63375 104.61625) (width 0.2) (layer "F.Cu") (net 10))
 (segment (start 102.63375 104.61625) (end 107.75 99.5) (width 0.2) (layer "F.Cu") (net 10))
 (segment (start 119.25 40.75) (end 115.75 37.25) (width 0.2) (layer "F.Cu") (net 10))
 (segment (start 115.5115 37.4885) (end 98.22 37.4885) (width 0.2) (layer "F.Cu") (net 10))
 (segment (start 115.75 99.5) (end 119.25 96) (width 0.2) (layer "F.Cu") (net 10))
 (segment (start 119.25 96) (end 119.25 40.75) (width 0.2) (layer "F.Cu") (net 10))
 (segment (start 120.25 97) (end 120.25 38) (width 0.2) (layer "F.Cu") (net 2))
 (segment (start 112.63375 104.61625) (end 120.25 97) (width 0.2) (layer "F.Cu") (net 2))
 (segment (start 120.25 38) (end 117.1985 34.9485) (width 0.2) (layer "F.Cu") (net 2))
 (segment (start 105.7275 104.61625) (end 112.63375 104.61625) (width 0.2) (layer "F.Cu") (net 2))
 (segment (start 117.1985 34.9485) (end 99.055 34.9485) (width 0.2) (layer "F.Cu") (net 2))
 (segment (start 82.25 96.75) (end 82.25 107.25) (width 0.2) (layer "F.Cu") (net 11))
 (segment (start 82 96.5) (end 82.25 96.75) (width 0.2) (layer "F.Cu") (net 11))
 (segment (start 117.25 103.5) (end 120.651 100.099) (width 0.2) (layer "F.Cu") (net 11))
 (segment (start 115.5 31.5) (end 114.5915 32.4085) (width 0.2) (layer "F.Cu") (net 11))
 (segment (start 120.651 100.099) (end 120.651 36.651) (width 0.2) (layer "F.Cu") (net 11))
 (segment (start 86.25 111.25) (end 115.75 111.25) (width 0.2) (layer "F.Cu") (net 11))
 (segment (start 115.75 111.25) (end 117.5 109.5) (width 0.2) (layer "F.Cu") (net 11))
 (segment (start 64.3125 95.5625) (end 65.25 96.5) (width 0.2) (layer "F.Cu") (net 11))
 (segment (start 82.25 107.25) (end 86.25 111.25) (width 0.2) (layer "F.Cu") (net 11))
 (segment (start 114.5915 32.4085) (end 99.055 32.4085) (width 0.2) (layer "F.Cu") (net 11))
 (segment (start 117.5 103.75) (end 117.25 103.5) (width 0.2) (layer "F.Cu") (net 11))
 (segment (start 65.25 96.5) (end 82 96.5) (width 0.2) (layer "F.Cu") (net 11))
 (segment (start 117.5 109.5) (end 117.5 103.75) (width 0.2) (layer "F.Cu") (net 11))
 (segment (start 120.651 36.651) (end 115.5 31.5) (width 0.2) (layer "F.Cu") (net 11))
 (segment (start 64.3125 90.60625) (end 64.3125 95.5625) (width 0.2) (layer "F.Cu") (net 11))
 (segment (start 95.6 32.4885) (end 98.22 29.8685) (width 0.2) (layer "F.Cu") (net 12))
 (segment (start 115.2 39.6) (end 95.7 39.6) (width 0.2) (layer "F.Cu") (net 12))
 (segment (start 66.6 80.2) (end 112.4 80.2) (width 0.2) (layer "F.Cu") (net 12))
 (segment (start 117.9 42.3) (end 115.2 39.6) (width 0.2) (layer "F.Cu") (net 12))
 (segment (start 95.6 39.5) (end 95.6 32.4885) (width 0.2) (layer "F.Cu") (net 12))
 (segment (start 64.3125 85.60625) (end 64.3125 82.4875) (width 0.2) (layer "F.Cu") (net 12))
 (segment (start 95.7 39.6) (end 95.6 39.5) (width 0.2) (layer "F.Cu") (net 12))
 (segment (start 112.4 80.2) (end 117.9 74.7) (width 0.2) (layer "F.Cu") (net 12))
 (segment (start 64.3125 82.4875) (end 66.6 80.2) (width 0.2) (layer "F.Cu") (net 12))
 (segment (start 117.9 74.7) (end 117.9 42.3) (width 0.2) (layer "F.Cu") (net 12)))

